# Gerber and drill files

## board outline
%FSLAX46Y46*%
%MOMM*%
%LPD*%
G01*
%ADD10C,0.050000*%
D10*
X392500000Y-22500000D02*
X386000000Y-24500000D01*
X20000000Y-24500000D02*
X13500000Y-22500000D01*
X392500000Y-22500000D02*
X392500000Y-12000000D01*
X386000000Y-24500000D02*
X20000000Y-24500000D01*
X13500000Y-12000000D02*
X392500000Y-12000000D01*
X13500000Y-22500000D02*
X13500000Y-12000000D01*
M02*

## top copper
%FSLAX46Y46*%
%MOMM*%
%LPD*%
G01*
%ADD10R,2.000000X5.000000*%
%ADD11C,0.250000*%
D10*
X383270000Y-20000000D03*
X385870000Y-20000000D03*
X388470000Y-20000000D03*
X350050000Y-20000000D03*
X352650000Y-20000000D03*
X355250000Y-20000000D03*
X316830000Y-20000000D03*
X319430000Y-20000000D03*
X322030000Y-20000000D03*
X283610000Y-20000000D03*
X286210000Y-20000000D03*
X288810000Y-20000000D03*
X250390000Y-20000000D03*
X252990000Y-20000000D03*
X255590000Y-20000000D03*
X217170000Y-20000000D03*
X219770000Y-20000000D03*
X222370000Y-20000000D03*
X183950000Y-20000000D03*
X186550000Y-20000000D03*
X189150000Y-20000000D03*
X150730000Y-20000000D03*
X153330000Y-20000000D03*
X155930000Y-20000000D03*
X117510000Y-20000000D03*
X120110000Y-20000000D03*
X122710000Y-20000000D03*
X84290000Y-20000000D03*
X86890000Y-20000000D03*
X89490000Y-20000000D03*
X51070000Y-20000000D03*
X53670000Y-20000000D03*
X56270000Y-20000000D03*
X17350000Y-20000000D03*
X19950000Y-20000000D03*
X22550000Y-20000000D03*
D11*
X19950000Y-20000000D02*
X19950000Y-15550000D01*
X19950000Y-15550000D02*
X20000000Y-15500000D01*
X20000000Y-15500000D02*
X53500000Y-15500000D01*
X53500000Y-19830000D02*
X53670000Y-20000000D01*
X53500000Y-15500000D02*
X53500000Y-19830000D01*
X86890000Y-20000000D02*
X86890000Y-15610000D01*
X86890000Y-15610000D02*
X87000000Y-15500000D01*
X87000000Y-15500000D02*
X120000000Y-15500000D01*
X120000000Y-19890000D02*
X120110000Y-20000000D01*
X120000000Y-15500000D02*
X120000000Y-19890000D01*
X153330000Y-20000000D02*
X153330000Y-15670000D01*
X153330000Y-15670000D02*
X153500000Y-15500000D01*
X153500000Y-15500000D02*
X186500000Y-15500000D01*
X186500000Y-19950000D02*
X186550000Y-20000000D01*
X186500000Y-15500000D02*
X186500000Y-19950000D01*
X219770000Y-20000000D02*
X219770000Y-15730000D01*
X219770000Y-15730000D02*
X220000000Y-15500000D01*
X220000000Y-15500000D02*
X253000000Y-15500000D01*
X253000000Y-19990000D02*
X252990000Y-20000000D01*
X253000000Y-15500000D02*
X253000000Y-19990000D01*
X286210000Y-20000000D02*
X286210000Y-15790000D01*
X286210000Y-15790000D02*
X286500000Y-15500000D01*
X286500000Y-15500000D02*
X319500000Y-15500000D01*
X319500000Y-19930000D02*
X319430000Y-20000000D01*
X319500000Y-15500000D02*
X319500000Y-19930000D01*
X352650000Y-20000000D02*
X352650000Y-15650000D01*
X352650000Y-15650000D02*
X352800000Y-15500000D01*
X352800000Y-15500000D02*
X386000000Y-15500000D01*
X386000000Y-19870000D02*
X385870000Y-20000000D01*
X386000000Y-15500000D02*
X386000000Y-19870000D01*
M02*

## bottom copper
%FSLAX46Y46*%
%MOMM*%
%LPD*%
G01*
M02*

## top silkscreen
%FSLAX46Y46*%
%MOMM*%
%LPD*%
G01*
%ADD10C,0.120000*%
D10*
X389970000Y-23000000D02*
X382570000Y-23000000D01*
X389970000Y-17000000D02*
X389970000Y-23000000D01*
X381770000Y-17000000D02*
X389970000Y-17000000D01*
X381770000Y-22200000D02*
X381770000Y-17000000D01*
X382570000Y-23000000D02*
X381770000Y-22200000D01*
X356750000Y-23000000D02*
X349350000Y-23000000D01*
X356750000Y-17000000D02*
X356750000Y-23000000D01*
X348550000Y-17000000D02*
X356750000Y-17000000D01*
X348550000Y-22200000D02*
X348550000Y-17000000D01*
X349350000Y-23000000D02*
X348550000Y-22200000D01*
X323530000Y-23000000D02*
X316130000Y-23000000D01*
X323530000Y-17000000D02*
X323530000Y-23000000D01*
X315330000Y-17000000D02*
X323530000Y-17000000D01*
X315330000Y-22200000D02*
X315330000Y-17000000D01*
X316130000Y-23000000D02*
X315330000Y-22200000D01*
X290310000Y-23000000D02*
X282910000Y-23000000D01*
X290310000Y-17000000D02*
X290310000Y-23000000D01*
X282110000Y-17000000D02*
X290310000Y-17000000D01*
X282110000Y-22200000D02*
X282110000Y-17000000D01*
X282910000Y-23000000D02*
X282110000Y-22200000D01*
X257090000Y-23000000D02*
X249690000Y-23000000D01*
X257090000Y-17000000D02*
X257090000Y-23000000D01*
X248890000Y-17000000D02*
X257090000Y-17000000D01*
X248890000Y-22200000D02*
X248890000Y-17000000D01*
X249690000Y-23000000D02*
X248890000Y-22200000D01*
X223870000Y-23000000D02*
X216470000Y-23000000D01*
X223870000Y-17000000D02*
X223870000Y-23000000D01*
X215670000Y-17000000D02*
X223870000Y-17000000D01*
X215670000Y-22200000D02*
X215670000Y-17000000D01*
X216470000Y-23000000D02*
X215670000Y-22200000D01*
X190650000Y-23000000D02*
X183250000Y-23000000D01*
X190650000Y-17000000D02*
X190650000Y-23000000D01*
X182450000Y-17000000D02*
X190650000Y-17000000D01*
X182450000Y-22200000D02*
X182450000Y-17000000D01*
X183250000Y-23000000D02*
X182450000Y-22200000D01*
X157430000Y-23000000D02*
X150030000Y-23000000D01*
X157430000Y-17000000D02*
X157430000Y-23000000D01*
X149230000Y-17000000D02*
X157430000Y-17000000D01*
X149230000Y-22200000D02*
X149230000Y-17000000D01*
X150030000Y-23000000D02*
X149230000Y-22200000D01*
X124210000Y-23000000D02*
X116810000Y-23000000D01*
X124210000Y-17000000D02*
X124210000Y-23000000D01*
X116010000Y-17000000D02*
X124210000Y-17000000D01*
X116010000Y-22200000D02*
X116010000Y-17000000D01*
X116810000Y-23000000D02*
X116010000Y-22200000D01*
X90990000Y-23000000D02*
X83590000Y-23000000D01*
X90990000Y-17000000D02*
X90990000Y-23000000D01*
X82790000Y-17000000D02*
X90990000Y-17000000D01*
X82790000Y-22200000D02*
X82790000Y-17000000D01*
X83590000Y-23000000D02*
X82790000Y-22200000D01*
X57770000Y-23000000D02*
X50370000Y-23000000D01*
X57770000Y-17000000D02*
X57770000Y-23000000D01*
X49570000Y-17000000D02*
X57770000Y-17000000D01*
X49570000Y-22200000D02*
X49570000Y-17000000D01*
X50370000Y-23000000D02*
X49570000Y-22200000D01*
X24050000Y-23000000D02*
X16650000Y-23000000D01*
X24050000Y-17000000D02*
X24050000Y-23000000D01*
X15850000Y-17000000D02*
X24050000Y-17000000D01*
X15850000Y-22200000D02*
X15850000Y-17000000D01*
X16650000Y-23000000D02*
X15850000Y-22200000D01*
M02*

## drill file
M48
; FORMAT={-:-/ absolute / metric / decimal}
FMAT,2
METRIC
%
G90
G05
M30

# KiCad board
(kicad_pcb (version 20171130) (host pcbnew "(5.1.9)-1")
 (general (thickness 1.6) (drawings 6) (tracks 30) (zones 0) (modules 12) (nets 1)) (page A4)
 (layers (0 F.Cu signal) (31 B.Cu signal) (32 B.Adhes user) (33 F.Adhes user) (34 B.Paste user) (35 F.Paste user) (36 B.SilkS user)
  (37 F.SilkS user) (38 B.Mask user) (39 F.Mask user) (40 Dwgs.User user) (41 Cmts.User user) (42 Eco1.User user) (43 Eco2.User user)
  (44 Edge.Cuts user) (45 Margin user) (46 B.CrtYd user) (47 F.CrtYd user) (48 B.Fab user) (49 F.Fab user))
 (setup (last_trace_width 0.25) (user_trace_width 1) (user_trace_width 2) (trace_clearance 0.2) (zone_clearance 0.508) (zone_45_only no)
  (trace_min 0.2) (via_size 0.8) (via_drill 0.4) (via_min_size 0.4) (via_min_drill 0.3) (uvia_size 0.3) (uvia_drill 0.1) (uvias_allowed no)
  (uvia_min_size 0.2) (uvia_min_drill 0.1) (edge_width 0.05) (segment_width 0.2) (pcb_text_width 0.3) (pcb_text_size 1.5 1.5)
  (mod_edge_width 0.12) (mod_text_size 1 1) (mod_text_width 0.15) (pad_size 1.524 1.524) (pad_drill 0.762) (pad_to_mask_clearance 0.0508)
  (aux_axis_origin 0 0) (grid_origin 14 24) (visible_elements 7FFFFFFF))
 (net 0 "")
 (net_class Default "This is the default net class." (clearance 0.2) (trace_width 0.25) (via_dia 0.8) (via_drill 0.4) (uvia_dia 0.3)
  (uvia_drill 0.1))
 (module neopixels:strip (layer F.Cu) (at 385.87 20)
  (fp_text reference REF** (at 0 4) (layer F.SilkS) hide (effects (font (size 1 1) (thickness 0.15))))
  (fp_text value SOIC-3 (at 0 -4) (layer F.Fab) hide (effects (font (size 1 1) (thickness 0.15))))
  (fp_line (start 4.1 3) (end -3.3 3) (layer F.SilkS) (width 0.12))
  (fp_line (start 4.1 -3) (end 4.1 3) (layer F.SilkS) (width 0.12))
  (fp_line (start -4.1 -3) (end 4.1 -3) (layer F.SilkS) (width 0.12))
  (fp_line (start -4.1 2.2) (end -4.1 -3) (layer F.SilkS) (width 0.12))
  (fp_line (start -3.3 3) (end -4.1 2.2) (layer F.SilkS) (width 0.12))
  (pad 1 smd rect (at -2.6 0) (size 2 5) (layers F.Cu F.Paste F.Mask))
  (pad 2 smd rect (at 0 0) (size 2 5) (layers F.Cu F.Paste F.Mask))
  (pad 3 smd rect (at 2.6 0) (size 2 5) (layers F.Cu F.Paste F.Mask)))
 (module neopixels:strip (layer F.Cu) (at 352.65 20)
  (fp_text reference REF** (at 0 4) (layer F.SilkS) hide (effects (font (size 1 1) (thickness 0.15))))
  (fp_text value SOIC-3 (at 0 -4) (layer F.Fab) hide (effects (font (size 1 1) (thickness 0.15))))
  (fp_line (start 4.1 3) (end -3.3 3) (layer F.SilkS) (width 0.12))
  (fp_line (start 4.1 -3) (end 4.1 3) (layer F.SilkS) (width 0.12))
  (fp_line (start -4.1 -3) (end 4.1 -3) (layer F.SilkS) (width 0.12))
  (fp_line (start -4.1 2.2) (end -4.1 -3) (layer F.SilkS) (width 0.12))
  (fp_line (start -3.3 3) (end -4.1 2.2) (layer F.SilkS) (width 0.12))
  (pad 1 smd rect (at -2.6 0) (size 2 5) (layers F.Cu F.Paste F.Mask))
  (pad 2 smd rect (at 0 0) (size 2 5) (layers F.Cu F.Paste F.Mask))
  (pad 3 smd rect (at 2.6 0) (size 2 5) (layers F.Cu F.Paste F.Mask)))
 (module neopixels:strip (layer F.Cu) (at 319.43 20)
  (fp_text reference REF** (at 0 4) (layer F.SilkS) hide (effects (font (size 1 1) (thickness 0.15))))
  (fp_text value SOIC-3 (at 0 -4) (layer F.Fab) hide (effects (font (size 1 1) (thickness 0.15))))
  (fp_line (start 4.1 3) (end -3.3 3) (layer F.SilkS) (width 0.12))
  (fp_line (start 4.1 -3) (end 4.1 3) (layer F.SilkS) (width 0.12))
  (fp_line (start -4.1 -3) (end 4.1 -3) (layer F.SilkS) (width 0.12))
  (fp_line (start -4.1 2.2) (end -4.1 -3) (layer F.SilkS) (width 0.12))
  (fp_line (start -3.3 3) (end -4.1 2.2) (layer F.SilkS) (width 0.12))
  (pad 1 smd rect (at -2.6 0) (size 2 5) (layers F.Cu F.Paste F.Mask))
  (pad 2 smd rect (at 0 0) (size 2 5) (layers F.Cu F.Paste F.Mask))
  (pad 3 smd rect (at 2.6 0) (size 2 5) (layers F.Cu F.Paste F.Mask)))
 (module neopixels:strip (layer F.Cu) (at 286.21 20)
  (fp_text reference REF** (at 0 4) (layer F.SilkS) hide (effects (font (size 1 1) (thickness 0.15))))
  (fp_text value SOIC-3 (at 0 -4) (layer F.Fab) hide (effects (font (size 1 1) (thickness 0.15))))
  (fp_line (start 4.1 3) (end -3.3 3) (layer F.SilkS) (width 0.12))
  (fp_line (start 4.1 -3) (end 4.1 3) (layer F.SilkS) (width 0.12))
  (fp_line (start -4.1 -3) (end 4.1 -3) (layer F.SilkS) (width 0.12))
  (fp_line (start -4.1 2.2) (end -4.1 -3) (layer F.SilkS) (width 0.12))
  (fp_line (start -3.3 3) (end -4.1 2.2) (layer F.SilkS) (width 0.12))
  (pad 1 smd rect (at -2.6 0) (size 2 5) (layers F.Cu F.Paste F.Mask))
  (pad 2 smd rect (at 0 0) (size 2 5) (layers F.Cu F.Paste F.Mask))
  (pad 3 smd rect (at 2.6 0) (size 2 5) (layers F.Cu F.Paste F.Mask)))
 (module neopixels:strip (layer F.Cu) (at 252.99 20)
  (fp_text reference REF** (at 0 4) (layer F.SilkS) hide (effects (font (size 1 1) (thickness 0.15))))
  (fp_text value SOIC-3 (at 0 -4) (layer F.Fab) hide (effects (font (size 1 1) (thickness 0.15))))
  (fp_line (start 4.1 3) (end -3.3 3) (layer F.SilkS) (width 0.12))
  (fp_line (start 4.1 -3) (end 4.1 3) (layer F.SilkS) (width 0.12))
  (fp_line (start -4.1 -3) (end 4.1 -3) (layer F.SilkS) (width 0.12))
  (fp_line (start -4.1 2.2) (end -4.1 -3) (layer F.SilkS) (width 0.12))
  (fp_line (start -3.3 3) (end -4.1 2.2) (layer F.SilkS) (width 0.12))
  (pad 1 smd rect (at -2.6 0) (size 2 5) (layers F.Cu F.Paste F.Mask))
  (pad 2 smd rect (at 0 0) (size 2 5) (layers F.Cu F.Paste F.Mask))
  (pad 3 smd rect (at 2.6 0) (size 2 5) (layers F.Cu F.Paste F.Mask)))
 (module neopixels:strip (layer F.Cu) (at 219.77 20)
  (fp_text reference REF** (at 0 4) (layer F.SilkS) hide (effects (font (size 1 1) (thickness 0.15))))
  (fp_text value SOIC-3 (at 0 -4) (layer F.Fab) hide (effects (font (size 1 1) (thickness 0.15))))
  (fp_line (start 4.1 3) (end -3.3 3) (layer F.SilkS) (width 0.12))
  (fp_line (start 4.1 -3) (end 4.1 3) (layer F.SilkS) (width 0.12))
  (fp_line (start -4.1 -3) (end 4.1 -3) (layer F.SilkS) (width 0.12))
  (fp_line (start -4.1 2.2) (end -4.1 -3) (layer F.SilkS) (width 0.12))
  (fp_line (start -3.3 3) (end -4.1 2.2) (layer F.SilkS) (width 0.12))
  (pad 1 smd rect (at -2.6 0) (size 2 5) (layers F.Cu F.Paste F.Mask))
  (pad 2 smd rect (at 0 0) (size 2 5) (layers F.Cu F.Paste F.Mask))
  (pad 3 smd rect (at 2.6 0) (size 2 5) (layers F.Cu F.Paste F.Mask)))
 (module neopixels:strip (layer F.Cu) (at 186.55 20)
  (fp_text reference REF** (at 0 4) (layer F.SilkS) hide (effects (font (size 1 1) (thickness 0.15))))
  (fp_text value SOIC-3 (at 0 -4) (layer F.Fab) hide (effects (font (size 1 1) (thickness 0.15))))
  (fp_line (start 4.1 3) (end -3.3 3) (layer F.SilkS) (width 0.12))
  (fp_line (start 4.1 -3) (end 4.1 3) (layer F.SilkS) (width 0.12))
  (fp_line (start -4.1 -3) (end 4.1 -3) (layer F.SilkS) (width 0.12))
  (fp_line (start -4.1 2.2) (end -4.1 -3) (layer F.SilkS) (width 0.12))
  (fp_line (start -3.3 3) (end -4.1 2.2) (layer F.SilkS) (width 0.12))
  (pad 1 smd rect (at -2.6 0) (size 2 5) (layers F.Cu F.Paste F.Mask))
  (pad 2 smd rect (at 0 0) (size 2 5) (layers F.Cu F.Paste F.Mask))
  (pad 3 smd rect (at 2.6 0) (size 2 5) (layers F.Cu F.Paste F.Mask)))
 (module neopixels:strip (layer F.Cu) (at 153.33 20)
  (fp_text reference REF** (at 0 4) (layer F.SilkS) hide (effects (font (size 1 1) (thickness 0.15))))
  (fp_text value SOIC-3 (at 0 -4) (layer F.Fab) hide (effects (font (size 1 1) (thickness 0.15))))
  (fp_line (start 4.1 3) (end -3.3 3) (layer F.SilkS) (width 0.12))
  (fp_line (start 4.1 -3) (end 4.1 3) (layer F.SilkS) (width 0.12))
  (fp_line (start -4.1 -3) (end 4.1 -3) (layer F.SilkS) (width 0.12))
  (fp_line (start -4.1 2.2) (end -4.1 -3) (layer F.SilkS) (width 0.12))
  (fp_line (start -3.3 3) (end -4.1 2.2) (layer F.SilkS) (width 0.12))
  (pad 1 smd rect (at -2.6 0) (size 2 5) (layers F.Cu F.Paste F.Mask))
  (pad 2 smd rect (at 0 0) (size 2 5) (layers F.Cu F.Paste F.Mask))
  (pad 3 smd rect (at 2.6 0) (size 2 5) (layers F.Cu F.Paste F.Mask)))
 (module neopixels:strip (layer F.Cu) (at 120.11 20)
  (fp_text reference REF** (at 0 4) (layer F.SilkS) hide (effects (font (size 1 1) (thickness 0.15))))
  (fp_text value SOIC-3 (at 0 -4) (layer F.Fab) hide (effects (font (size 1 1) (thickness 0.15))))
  (fp_line (start 4.1 3) (end -3.3 3) (layer F.SilkS) (width 0.12))
  (fp_line (start 4.1 -3) (end 4.1 3) (layer F.SilkS) (width 0.12))
  (fp_line (start -4.1 -3) (end 4.1 -3) (layer F.SilkS) (width 0.12))
  (fp_line (start -4.1 2.2) (end -4.1 -3) (layer F.SilkS) (width 0.12))
  (fp_line (start -3.3 3) (end -4.1 2.2) (layer F.SilkS) (width 0.12))
  (pad 1 smd rect (at -2.6 0) (size 2 5) (layers F.Cu F.Paste F.Mask))
  (pad 2 smd rect (at 0 0) (size 2 5) (layers F.Cu F.Paste F.Mask))
  (pad 3 smd rect (at 2.6 0) (size 2 5) (layers F.Cu F.Paste F.Mask)))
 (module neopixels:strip (layer F.Cu) (at 86.89 20)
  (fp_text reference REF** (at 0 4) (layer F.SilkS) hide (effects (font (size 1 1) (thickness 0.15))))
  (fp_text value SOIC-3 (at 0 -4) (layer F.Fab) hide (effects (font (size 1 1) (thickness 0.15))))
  (fp_line (start 4.1 3) (end -3.3 3) (layer F.SilkS) (width 0.12))
  (fp_line (start 4.1 -3) (end 4.1 3) (layer F.SilkS) (width 0.12))
  (fp_line (start -4.1 -3) (end 4.1 -3) (layer F.SilkS) (width 0.12))
  (fp_line (start -4.1 2.2) (end -4.1 -3) (layer F.SilkS) (width 0.12))
  (fp_line (start -3.3 3) (end -4.1 2.2) (layer F.SilkS) (width 0.12))
  (pad 1 smd rect (at -2.6 0) (size 2 5) (layers F.Cu F.Paste F.Mask))
  (pad 2 smd rect (at 0 0) (size 2 5) (layers F.Cu F.Paste F.Mask))
  (pad 3 smd rect (at 2.6 0) (size 2 5) (layers F.Cu F.Paste F.Mask)))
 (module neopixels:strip (layer F.Cu) (at 53.67 20)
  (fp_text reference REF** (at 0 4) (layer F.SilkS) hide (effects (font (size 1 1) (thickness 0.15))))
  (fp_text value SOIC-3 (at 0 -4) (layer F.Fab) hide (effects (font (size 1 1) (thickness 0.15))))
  (fp_line (start 4.1 3) (end -3.3 3) (layer F.SilkS) (width 0.12))
  (fp_line (start 4.1 -3) (end 4.1 3) (layer F.SilkS) (width 0.12))
  (fp_line (start -4.1 -3) (end 4.1 -3) (layer F.SilkS) (width 0.12))
  (fp_line (start -4.1 2.2) (end -4.1 -3) (layer F.SilkS) (width 0.12))
  (fp_line (start -3.3 3) (end -4.1 2.2) (layer F.SilkS) (width 0.12))
  (pad 1 smd rect (at -2.6 0) (size 2 5) (layers F.Cu F.Paste F.Mask))
  (pad 2 smd rect (at 0 0) (size 2 5) (layers F.Cu F.Paste F.Mask))
  (pad 3 smd rect (at 2.6 0) (size 2 5) (layers F.Cu F.Paste F.Mask)))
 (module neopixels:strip (layer F.Cu) (at 19.95 20)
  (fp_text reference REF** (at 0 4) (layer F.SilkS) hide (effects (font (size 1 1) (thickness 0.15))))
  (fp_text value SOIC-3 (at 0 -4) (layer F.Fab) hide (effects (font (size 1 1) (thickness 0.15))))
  (fp_line (start 4.1 3) (end -3.3 3) (layer F.SilkS) (width 0.12))
  (fp_line (start 4.1 -3) (end 4.1 3) (layer F.SilkS) (width 0.12))
  (fp_line (start -4.1 -3) (end 4.1 -3) (layer F.SilkS) (width 0.12))
  (fp_line (start -4.1 2.2) (end -4.1 -3) (layer F.SilkS) (width 0.12))
  (fp_line (start -3.3 3) (end -4.1 2.2) (layer F.SilkS) (width 0.12))
  (pad 1 smd rect (at -2.6 0) (size 2 5) (layers F.Cu F.Paste F.Mask))
  (pad 2 smd rect (at 0 0) (size 2 5) (layers F.Cu F.Paste F.Mask))
  (pad 3 smd rect (at 2.6 0) (size 2 5) (layers F.Cu F.Paste F.Mask)))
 (gr_line (start 392.5 22.5) (end 386 24.5) (layer Edge.Cuts) (width 0.05))
 (gr_line (start 20 24.5) (end 13.5 22.5) (layer Edge.Cuts) (width 0.05))
 (gr_line (start 392.5 22.5) (end 392.5 12) (layer Edge.Cuts) (width 0.05))
 (gr_line (start 386 24.5) (end 20 24.5) (layer Edge.Cuts) (width 0.05))
 (gr_line (start 13.5 12) (end 392.5 12) (layer Edge.Cuts) (width 0.05))
 (gr_line (start 13.5 22.5) (end 13.5 12) (layer Edge.Cuts) (width 0.05))
 (segment (start 19.95 20) (end 19.95 15.55) (width 0.25) (layer F.Cu) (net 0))
 (segment (start 19.95 15.55) (end 20 15.5) (width 0.25) (layer F.Cu) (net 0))
 (segment (start 20 15.5) (end 53.5 15.5) (width 0.25) (layer F.Cu) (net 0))
 (segment (start 53.5 19.83) (end 53.67 20) (width 0.25) (layer F.Cu) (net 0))
 (segment (start 53.5 15.5) (end 53.5 19.83) (width 0.25) (layer F.Cu) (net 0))
 (segment (start 86.89 20) (end 86.89 15.61) (width 0.25) (layer F.Cu) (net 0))
 (segment (start 86.89 15.61) (end 87 15.5) (width 0.25) (layer F.Cu) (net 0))
 (segment (start 87 15.5) (end 120 15.5) (width 0.25) (layer F.Cu) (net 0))
 (segment (start 120 19.89) (end 120.11 20) (width 0.25) (layer F.Cu) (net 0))
 (segment (start 120 15.5) (end 120 19.89) (width 0.25) (layer F.Cu) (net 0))
 (segment (start 153.33 20) (end 153.33 15.67) (width 0.25) (layer F.Cu) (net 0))
 (segment (start 153.33 15.67) (end 153.5 15.5) (width 0.25) (layer F.Cu) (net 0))
 (segment (start 153.5 15.5) (end 186.5 15.5) (width 0.25) (layer F.Cu) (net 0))
 (segment (start 186.5 19.95) (end 186.55 20) (width 0.25) (layer F.Cu) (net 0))
 (segment (start 186.5 15.5) (end 186.5 19.95) (width 0.25) (layer F.Cu) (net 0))
 (segment (start 219.77 20) (end 219.77 15.73) (width 0.25) (layer F.Cu) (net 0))
 (segment (start 219.77 15.73) (end 220 15.5) (width 0.25) (layer F.Cu) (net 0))
 (segment (start 220 15.5) (end 253 15.5) (width 0.25) (layer F.Cu) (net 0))
 (segment (start 253 19.99) (end 252.99 20) (width 0.25) (layer F.Cu) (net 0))
 (segment (start 253 15.5) (end 253 19.99) (width 0.25) (layer F.Cu) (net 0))
 (segment (start 286.21 20) (end 286.21 15.79) (width 0.25) (layer F.Cu) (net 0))
 (segment (start 286.21 15.79) (end 286.5 15.5) (width 0.25) (layer F.Cu) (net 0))
 (segment (start 286.5 15.5) (end 319.5 15.5) (width 0.25) (layer F.Cu) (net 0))
 (segment (start 319.5 19.93) (end 319.43 20) (width 0.25) (layer F.Cu) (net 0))
 (segment (start 319.5 15.5) (end 319.5 19.93) (width 0.25) (layer F.Cu) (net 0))
 (segment (start 352.65 20) (end 352.65 15.65) (width 0.25) (layer F.Cu) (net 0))
 (segment (start 352.65 15.65) (end 352.8 15.5) (width 0.25) (layer F.Cu) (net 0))
 (segment (start 352.8 15.5) (end 386 15.5) (width 0.25) (layer F.Cu) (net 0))
 (segment (start 386 19.87) (end 385.87 20) (width 0.25) (layer F.Cu) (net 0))
 (segment (start 386 15.5) (end 386 19.87) (width 0.25) (layer F.Cu) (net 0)))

